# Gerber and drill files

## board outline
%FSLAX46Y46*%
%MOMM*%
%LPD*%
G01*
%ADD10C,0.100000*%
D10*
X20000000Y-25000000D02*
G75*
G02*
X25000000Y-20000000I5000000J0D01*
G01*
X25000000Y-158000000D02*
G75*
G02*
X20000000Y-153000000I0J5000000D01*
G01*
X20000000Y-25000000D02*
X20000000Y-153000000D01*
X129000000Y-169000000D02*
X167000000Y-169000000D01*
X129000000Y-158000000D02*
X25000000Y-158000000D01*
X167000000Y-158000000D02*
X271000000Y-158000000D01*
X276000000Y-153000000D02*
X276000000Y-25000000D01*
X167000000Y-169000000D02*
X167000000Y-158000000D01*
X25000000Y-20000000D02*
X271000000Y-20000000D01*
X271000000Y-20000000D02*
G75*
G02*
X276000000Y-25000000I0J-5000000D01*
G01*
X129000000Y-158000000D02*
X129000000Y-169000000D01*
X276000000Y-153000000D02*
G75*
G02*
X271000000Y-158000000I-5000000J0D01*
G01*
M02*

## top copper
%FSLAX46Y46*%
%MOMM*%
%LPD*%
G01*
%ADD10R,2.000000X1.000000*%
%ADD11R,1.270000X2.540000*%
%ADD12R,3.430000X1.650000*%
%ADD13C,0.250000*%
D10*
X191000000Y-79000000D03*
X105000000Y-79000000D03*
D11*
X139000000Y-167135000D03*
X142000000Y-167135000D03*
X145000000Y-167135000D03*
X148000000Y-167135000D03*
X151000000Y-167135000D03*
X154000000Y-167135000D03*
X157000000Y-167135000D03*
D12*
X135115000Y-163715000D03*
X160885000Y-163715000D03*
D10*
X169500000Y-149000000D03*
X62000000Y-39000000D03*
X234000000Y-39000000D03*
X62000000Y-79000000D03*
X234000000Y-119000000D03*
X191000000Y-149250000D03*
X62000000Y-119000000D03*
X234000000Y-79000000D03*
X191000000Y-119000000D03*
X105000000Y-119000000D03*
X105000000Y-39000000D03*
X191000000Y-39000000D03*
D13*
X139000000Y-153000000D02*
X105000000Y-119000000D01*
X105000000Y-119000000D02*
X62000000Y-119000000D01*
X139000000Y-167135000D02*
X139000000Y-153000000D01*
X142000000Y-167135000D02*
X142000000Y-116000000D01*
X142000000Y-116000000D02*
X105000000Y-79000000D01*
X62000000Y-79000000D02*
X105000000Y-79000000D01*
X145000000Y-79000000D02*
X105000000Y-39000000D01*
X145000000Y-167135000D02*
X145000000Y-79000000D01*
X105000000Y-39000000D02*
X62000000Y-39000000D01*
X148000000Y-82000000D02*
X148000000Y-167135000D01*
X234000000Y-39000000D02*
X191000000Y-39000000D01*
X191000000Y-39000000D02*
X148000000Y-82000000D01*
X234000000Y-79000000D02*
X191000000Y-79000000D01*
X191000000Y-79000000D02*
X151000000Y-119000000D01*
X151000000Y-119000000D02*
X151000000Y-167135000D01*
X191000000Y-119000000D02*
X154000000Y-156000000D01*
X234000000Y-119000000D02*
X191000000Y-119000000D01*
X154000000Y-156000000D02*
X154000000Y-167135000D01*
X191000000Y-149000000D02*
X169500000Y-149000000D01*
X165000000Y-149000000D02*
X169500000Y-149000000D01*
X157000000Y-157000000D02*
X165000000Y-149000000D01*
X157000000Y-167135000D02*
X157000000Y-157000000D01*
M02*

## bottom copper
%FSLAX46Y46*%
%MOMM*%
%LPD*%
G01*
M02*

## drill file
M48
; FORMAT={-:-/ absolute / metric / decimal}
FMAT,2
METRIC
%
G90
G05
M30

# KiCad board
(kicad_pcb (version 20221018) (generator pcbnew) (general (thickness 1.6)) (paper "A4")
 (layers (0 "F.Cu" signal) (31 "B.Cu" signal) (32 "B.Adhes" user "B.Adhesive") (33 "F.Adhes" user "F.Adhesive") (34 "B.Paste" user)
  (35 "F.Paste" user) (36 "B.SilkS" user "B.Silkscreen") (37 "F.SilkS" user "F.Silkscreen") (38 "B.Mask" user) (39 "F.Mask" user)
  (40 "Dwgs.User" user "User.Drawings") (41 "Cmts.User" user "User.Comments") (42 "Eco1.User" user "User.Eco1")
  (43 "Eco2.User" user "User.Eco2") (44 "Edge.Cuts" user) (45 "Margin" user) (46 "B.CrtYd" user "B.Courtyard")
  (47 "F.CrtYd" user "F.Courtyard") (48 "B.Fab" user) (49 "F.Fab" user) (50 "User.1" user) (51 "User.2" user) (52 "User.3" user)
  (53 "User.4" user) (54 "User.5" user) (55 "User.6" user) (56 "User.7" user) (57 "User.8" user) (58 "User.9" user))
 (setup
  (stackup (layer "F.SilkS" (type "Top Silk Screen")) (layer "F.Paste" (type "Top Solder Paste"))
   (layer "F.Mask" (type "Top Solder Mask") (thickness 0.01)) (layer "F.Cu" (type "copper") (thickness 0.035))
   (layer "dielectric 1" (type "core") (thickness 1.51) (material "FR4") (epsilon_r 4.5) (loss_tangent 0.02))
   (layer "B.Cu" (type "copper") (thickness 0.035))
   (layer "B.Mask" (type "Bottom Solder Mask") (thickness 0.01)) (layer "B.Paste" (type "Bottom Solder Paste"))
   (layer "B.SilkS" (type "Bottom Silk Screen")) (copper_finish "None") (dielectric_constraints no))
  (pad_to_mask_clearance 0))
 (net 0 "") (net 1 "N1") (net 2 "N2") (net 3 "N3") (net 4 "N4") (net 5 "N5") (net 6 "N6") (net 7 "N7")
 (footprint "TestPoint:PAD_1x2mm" (layer "F.Cu") (at 191 79)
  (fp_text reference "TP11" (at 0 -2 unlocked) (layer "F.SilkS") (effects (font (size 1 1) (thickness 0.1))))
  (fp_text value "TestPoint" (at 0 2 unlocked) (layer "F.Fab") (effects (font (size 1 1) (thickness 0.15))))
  (pad "1" smd rect (at 0 0 90) (size 1 2) (layers "F.Cu" "F.Paste" "F.Mask") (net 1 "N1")))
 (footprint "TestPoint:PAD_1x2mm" (layer "F.Cu") (at 105 79)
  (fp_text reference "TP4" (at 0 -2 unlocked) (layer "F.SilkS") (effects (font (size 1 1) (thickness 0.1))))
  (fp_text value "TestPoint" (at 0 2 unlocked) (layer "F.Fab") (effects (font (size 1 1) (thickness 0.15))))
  (pad "1" smd rect (at 0 0 90) (size 1 2) (layers "F.Cu" "F.Paste" "F.Mask") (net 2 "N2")))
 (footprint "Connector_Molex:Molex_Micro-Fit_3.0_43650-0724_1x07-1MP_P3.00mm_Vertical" (layer "F.Cu") (at 148 164)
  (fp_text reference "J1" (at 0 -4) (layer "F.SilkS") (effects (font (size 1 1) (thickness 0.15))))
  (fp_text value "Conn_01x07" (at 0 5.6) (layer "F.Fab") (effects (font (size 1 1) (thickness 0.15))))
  (pad "1" smd rect (at -9 3.135) (size 1.27 2.54) (layers "F.Cu" "F.Paste" "F.Mask") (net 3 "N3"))
  (pad "2" smd rect (at -6 3.135) (size 1.27 2.54) (layers "F.Cu" "F.Paste" "F.Mask") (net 2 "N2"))
  (pad "3" smd rect (at -3 3.135) (size 1.27 2.54) (layers "F.Cu" "F.Paste" "F.Mask") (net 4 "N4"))
  (pad "4" smd rect (at 0 3.135) (size 1.27 2.54) (layers "F.Cu" "F.Paste" "F.Mask") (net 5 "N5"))
  (pad "5" smd rect (at 3 3.135) (size 1.27 2.54) (layers "F.Cu" "F.Paste" "F.Mask") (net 1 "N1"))
  (pad "6" smd rect (at 6 3.135) (size 1.27 2.54) (layers "F.Cu" "F.Paste" "F.Mask") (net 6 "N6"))
  (pad "7" smd rect (at 9 3.135) (size 1.27 2.54) (layers "F.Cu" "F.Paste" "F.Mask") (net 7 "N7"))
  (pad "MP" smd rect (at -12.885 -0.285) (size 3.43 1.65) (layers "F.Cu" "F.Paste" "F.Mask"))
  (pad "MP" smd rect (at 12.885 -0.285) (size 3.43 1.65) (layers "F.Cu" "F.Paste" "F.Mask")))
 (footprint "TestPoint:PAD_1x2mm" (layer "F.Cu") (at 169.5 149)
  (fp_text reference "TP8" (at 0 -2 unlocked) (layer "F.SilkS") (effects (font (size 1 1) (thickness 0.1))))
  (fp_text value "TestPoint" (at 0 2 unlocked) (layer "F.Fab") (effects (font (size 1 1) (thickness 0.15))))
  (pad "1" smd rect (at 0 0 90) (size 1 2) (layers "F.Cu" "F.Paste" "F.Mask") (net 7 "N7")))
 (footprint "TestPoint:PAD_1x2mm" (layer "F.Cu") (at 62 39)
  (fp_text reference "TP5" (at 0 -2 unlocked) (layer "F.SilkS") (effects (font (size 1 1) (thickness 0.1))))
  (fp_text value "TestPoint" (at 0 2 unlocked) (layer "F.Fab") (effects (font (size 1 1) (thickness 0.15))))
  (pad "1" smd rect (at 0 0 90) (size 1 2) (layers "F.Cu" "F.Paste" "F.Mask") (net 4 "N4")))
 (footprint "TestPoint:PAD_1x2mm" (layer "F.Cu") (at 234 39)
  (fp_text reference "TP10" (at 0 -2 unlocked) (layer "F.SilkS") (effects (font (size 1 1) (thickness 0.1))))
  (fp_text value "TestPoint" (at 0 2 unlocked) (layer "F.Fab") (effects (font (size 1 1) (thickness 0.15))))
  (pad "1" smd rect (at 0 0 90) (size 1 2) (layers "F.Cu" "F.Paste" "F.Mask") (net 5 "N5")))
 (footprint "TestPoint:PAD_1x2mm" (layer "F.Cu") (at 62 79)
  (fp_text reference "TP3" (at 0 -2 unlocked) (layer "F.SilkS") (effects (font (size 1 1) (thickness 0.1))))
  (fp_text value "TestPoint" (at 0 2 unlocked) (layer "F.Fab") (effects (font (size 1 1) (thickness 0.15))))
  (pad "1" smd rect (at 0 0 90) (size 1 2) (layers "F.Cu" "F.Paste" "F.Mask") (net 2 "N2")))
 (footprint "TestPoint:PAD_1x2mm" (layer "F.Cu") (at 234 119)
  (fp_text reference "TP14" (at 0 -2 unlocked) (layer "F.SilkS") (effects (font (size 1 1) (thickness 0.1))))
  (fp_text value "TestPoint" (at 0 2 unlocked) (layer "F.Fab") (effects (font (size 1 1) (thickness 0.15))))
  (pad "1" smd rect (at 0 0 90) (size 1 2) (layers "F.Cu" "F.Paste" "F.Mask") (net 6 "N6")))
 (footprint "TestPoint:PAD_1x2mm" (layer "F.Cu") (at 191 149.25)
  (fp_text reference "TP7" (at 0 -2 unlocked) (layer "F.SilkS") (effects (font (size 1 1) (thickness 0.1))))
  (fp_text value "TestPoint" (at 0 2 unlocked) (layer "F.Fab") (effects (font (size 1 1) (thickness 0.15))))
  (pad "1" smd rect (at 0 0 90) (size 1 2) (layers "F.Cu" "F.Paste" "F.Mask") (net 7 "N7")))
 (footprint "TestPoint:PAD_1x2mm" (layer "F.Cu") (at 62 119)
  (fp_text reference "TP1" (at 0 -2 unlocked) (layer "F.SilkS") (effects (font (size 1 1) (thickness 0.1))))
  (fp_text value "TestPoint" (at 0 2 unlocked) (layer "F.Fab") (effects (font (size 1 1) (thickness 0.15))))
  (pad "1" smd rect (at 0 0 90) (size 1 2) (layers "F.Cu" "F.Paste" "F.Mask") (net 3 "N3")))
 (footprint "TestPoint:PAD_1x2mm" (layer "F.Cu") (at 234 79)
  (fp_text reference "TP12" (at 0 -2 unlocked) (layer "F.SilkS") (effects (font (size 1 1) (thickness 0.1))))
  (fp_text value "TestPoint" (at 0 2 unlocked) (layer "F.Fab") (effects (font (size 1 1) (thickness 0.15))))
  (pad "1" smd rect (at 0 0 90) (size 1 2) (layers "F.Cu" "F.Paste" "F.Mask") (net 1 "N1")))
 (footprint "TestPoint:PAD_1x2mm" (layer "F.Cu") (at 191 119)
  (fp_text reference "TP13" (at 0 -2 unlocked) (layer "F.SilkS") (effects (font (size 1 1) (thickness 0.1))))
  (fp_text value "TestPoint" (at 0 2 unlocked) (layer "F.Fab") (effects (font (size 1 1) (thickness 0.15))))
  (pad "1" smd rect (at 0 0 90) (size 1 2) (layers "F.Cu" "F.Paste" "F.Mask") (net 6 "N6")))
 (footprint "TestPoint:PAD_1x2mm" (layer "F.Cu") (at 105 119)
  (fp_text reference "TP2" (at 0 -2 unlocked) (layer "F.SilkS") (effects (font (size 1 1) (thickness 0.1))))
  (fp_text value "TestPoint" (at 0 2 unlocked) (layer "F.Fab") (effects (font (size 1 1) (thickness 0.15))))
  (pad "1" smd rect (at 0 0 90) (size 1 2) (layers "F.Cu" "F.Paste" "F.Mask") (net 3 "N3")))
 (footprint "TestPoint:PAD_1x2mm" (layer "F.Cu") (at 105 39)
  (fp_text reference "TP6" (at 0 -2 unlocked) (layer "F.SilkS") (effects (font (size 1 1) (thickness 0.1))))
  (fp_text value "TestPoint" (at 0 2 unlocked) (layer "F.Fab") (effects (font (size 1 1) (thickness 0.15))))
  (pad "1" smd rect (at 0 0 90) (size 1 2) (layers "F.Cu" "F.Paste" "F.Mask") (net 4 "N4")))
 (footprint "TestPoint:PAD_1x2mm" (layer "F.Cu") (at 191 39)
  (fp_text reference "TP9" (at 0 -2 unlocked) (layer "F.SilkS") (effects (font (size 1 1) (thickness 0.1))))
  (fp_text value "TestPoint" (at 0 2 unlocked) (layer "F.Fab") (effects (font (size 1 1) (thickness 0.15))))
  (pad "1" smd rect (at 0 0 90) (size 1 2) (layers "F.Cu" "F.Paste" "F.Mask") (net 5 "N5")))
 (gr_arc (start 20 25) (mid 21.464466 21.464466) (end 25 20) (stroke (width 0.1) (type default)) (layer "Edge.Cuts"))
 (gr_arc (start 25 158) (mid 21.464466 156.535534) (end 20 153) (stroke (width 0.1) (type default)) (layer "Edge.Cuts"))
 (gr_line (start 20 25) (end 20 153) (stroke (width 0.1) (type default)) (layer "Edge.Cuts"))
 (gr_line (start 129 169) (end 167 169) (stroke (width 0.1) (type default)) (layer "Edge.Cuts"))
 (gr_line (start 129 158) (end 25 158) (stroke (width 0.1) (type default)) (layer "Edge.Cuts"))
 (gr_line (start 167 158) (end 271 158) (stroke (width 0.1) (type default)) (layer "Edge.Cuts"))
 (gr_line (start 276 153) (end 276 25) (stroke (width 0.1) (type default)) (layer "Edge.Cuts"))
 (gr_line (start 167 169) (end 167 158) (stroke (width 0.1) (type default)) (layer "Edge.Cuts"))
 (gr_line (start 25 20) (end 271 20) (stroke (width 0.1) (type default)) (layer "Edge.Cuts"))
 (gr_arc (start 271 20) (mid 274.535534 21.464466) (end 276 25) (stroke (width 0.1) (type default)) (layer "Edge.Cuts"))
 (gr_line (start 129 158) (end 129 169) (stroke (width 0.1) (type default)) (layer "Edge.Cuts"))
 (gr_arc (start 276 153) (mid 274.535534 156.535534) (end 271 158) (stroke (width 0.1) (type default)) (layer "Edge.Cuts"))
 (segment (start 139 153) (end 105 119) (width 0.25) (layer "F.Cu") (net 3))
 (segment (start 105 119) (end 62 119) (width 0.25) (layer "F.Cu") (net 3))
 (segment (start 139 167.135) (end 139 153) (width 0.25) (layer "F.Cu") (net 3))
 (segment (start 142 167.135) (end 142 116) (width 0.25) (layer "F.Cu") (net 2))
 (segment (start 142 116) (end 105 79) (width 0.25) (layer "F.Cu") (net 2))
 (segment (start 62 79) (end 105 79) (width 0.25) (layer "F.Cu") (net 2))
 (segment (start 145 79) (end 105 39) (width 0.25) (layer "F.Cu") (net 4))
 (segment (start 145 167.135) (end 145 79) (width 0.25) (layer "F.Cu") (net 4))
 (segment (start 105 39) (end 62 39) (width 0.25) (layer "F.Cu") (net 4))
 (segment (start 148 82) (end 148 167.135) (width 0.25) (layer "F.Cu") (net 5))
 (segment (start 234 39) (end 191 39) (width 0.25) (layer "F.Cu") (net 5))
 (segment (start 191 39) (end 148 82) (width 0.25) (layer "F.Cu") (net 5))
 (segment (start 234 79) (end 191 79) (width 0.25) (layer "F.Cu") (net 1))
 (segment (start 191 79) (end 151 119) (width 0.25) (layer "F.Cu") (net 1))
 (segment (start 151 119) (end 151 167.135) (width 0.25) (layer "F.Cu") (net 1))
 (segment (start 191 119) (end 154 156) (width 0.25) (layer "F.Cu") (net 6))
 (segment (start 234 119) (end 191 119) (width 0.25) (layer "F.Cu") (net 6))
 (segment (start 154 156) (end 154 167.135) (width 0.25) (layer "F.Cu") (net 6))
 (segment (start 191 149) (end 169.5 149) (width 0.25) (layer "F.Cu") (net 7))
 (segment (start 165 149) (end 169.5 149) (width 0.25) (layer "F.Cu") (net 7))
 (segment (start 157 157) (end 165 149) (width 0.25) (layer "F.Cu") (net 7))
 (segment (start 157 167.135) (end 157 157) (width 0.25) (layer "F.Cu") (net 7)))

